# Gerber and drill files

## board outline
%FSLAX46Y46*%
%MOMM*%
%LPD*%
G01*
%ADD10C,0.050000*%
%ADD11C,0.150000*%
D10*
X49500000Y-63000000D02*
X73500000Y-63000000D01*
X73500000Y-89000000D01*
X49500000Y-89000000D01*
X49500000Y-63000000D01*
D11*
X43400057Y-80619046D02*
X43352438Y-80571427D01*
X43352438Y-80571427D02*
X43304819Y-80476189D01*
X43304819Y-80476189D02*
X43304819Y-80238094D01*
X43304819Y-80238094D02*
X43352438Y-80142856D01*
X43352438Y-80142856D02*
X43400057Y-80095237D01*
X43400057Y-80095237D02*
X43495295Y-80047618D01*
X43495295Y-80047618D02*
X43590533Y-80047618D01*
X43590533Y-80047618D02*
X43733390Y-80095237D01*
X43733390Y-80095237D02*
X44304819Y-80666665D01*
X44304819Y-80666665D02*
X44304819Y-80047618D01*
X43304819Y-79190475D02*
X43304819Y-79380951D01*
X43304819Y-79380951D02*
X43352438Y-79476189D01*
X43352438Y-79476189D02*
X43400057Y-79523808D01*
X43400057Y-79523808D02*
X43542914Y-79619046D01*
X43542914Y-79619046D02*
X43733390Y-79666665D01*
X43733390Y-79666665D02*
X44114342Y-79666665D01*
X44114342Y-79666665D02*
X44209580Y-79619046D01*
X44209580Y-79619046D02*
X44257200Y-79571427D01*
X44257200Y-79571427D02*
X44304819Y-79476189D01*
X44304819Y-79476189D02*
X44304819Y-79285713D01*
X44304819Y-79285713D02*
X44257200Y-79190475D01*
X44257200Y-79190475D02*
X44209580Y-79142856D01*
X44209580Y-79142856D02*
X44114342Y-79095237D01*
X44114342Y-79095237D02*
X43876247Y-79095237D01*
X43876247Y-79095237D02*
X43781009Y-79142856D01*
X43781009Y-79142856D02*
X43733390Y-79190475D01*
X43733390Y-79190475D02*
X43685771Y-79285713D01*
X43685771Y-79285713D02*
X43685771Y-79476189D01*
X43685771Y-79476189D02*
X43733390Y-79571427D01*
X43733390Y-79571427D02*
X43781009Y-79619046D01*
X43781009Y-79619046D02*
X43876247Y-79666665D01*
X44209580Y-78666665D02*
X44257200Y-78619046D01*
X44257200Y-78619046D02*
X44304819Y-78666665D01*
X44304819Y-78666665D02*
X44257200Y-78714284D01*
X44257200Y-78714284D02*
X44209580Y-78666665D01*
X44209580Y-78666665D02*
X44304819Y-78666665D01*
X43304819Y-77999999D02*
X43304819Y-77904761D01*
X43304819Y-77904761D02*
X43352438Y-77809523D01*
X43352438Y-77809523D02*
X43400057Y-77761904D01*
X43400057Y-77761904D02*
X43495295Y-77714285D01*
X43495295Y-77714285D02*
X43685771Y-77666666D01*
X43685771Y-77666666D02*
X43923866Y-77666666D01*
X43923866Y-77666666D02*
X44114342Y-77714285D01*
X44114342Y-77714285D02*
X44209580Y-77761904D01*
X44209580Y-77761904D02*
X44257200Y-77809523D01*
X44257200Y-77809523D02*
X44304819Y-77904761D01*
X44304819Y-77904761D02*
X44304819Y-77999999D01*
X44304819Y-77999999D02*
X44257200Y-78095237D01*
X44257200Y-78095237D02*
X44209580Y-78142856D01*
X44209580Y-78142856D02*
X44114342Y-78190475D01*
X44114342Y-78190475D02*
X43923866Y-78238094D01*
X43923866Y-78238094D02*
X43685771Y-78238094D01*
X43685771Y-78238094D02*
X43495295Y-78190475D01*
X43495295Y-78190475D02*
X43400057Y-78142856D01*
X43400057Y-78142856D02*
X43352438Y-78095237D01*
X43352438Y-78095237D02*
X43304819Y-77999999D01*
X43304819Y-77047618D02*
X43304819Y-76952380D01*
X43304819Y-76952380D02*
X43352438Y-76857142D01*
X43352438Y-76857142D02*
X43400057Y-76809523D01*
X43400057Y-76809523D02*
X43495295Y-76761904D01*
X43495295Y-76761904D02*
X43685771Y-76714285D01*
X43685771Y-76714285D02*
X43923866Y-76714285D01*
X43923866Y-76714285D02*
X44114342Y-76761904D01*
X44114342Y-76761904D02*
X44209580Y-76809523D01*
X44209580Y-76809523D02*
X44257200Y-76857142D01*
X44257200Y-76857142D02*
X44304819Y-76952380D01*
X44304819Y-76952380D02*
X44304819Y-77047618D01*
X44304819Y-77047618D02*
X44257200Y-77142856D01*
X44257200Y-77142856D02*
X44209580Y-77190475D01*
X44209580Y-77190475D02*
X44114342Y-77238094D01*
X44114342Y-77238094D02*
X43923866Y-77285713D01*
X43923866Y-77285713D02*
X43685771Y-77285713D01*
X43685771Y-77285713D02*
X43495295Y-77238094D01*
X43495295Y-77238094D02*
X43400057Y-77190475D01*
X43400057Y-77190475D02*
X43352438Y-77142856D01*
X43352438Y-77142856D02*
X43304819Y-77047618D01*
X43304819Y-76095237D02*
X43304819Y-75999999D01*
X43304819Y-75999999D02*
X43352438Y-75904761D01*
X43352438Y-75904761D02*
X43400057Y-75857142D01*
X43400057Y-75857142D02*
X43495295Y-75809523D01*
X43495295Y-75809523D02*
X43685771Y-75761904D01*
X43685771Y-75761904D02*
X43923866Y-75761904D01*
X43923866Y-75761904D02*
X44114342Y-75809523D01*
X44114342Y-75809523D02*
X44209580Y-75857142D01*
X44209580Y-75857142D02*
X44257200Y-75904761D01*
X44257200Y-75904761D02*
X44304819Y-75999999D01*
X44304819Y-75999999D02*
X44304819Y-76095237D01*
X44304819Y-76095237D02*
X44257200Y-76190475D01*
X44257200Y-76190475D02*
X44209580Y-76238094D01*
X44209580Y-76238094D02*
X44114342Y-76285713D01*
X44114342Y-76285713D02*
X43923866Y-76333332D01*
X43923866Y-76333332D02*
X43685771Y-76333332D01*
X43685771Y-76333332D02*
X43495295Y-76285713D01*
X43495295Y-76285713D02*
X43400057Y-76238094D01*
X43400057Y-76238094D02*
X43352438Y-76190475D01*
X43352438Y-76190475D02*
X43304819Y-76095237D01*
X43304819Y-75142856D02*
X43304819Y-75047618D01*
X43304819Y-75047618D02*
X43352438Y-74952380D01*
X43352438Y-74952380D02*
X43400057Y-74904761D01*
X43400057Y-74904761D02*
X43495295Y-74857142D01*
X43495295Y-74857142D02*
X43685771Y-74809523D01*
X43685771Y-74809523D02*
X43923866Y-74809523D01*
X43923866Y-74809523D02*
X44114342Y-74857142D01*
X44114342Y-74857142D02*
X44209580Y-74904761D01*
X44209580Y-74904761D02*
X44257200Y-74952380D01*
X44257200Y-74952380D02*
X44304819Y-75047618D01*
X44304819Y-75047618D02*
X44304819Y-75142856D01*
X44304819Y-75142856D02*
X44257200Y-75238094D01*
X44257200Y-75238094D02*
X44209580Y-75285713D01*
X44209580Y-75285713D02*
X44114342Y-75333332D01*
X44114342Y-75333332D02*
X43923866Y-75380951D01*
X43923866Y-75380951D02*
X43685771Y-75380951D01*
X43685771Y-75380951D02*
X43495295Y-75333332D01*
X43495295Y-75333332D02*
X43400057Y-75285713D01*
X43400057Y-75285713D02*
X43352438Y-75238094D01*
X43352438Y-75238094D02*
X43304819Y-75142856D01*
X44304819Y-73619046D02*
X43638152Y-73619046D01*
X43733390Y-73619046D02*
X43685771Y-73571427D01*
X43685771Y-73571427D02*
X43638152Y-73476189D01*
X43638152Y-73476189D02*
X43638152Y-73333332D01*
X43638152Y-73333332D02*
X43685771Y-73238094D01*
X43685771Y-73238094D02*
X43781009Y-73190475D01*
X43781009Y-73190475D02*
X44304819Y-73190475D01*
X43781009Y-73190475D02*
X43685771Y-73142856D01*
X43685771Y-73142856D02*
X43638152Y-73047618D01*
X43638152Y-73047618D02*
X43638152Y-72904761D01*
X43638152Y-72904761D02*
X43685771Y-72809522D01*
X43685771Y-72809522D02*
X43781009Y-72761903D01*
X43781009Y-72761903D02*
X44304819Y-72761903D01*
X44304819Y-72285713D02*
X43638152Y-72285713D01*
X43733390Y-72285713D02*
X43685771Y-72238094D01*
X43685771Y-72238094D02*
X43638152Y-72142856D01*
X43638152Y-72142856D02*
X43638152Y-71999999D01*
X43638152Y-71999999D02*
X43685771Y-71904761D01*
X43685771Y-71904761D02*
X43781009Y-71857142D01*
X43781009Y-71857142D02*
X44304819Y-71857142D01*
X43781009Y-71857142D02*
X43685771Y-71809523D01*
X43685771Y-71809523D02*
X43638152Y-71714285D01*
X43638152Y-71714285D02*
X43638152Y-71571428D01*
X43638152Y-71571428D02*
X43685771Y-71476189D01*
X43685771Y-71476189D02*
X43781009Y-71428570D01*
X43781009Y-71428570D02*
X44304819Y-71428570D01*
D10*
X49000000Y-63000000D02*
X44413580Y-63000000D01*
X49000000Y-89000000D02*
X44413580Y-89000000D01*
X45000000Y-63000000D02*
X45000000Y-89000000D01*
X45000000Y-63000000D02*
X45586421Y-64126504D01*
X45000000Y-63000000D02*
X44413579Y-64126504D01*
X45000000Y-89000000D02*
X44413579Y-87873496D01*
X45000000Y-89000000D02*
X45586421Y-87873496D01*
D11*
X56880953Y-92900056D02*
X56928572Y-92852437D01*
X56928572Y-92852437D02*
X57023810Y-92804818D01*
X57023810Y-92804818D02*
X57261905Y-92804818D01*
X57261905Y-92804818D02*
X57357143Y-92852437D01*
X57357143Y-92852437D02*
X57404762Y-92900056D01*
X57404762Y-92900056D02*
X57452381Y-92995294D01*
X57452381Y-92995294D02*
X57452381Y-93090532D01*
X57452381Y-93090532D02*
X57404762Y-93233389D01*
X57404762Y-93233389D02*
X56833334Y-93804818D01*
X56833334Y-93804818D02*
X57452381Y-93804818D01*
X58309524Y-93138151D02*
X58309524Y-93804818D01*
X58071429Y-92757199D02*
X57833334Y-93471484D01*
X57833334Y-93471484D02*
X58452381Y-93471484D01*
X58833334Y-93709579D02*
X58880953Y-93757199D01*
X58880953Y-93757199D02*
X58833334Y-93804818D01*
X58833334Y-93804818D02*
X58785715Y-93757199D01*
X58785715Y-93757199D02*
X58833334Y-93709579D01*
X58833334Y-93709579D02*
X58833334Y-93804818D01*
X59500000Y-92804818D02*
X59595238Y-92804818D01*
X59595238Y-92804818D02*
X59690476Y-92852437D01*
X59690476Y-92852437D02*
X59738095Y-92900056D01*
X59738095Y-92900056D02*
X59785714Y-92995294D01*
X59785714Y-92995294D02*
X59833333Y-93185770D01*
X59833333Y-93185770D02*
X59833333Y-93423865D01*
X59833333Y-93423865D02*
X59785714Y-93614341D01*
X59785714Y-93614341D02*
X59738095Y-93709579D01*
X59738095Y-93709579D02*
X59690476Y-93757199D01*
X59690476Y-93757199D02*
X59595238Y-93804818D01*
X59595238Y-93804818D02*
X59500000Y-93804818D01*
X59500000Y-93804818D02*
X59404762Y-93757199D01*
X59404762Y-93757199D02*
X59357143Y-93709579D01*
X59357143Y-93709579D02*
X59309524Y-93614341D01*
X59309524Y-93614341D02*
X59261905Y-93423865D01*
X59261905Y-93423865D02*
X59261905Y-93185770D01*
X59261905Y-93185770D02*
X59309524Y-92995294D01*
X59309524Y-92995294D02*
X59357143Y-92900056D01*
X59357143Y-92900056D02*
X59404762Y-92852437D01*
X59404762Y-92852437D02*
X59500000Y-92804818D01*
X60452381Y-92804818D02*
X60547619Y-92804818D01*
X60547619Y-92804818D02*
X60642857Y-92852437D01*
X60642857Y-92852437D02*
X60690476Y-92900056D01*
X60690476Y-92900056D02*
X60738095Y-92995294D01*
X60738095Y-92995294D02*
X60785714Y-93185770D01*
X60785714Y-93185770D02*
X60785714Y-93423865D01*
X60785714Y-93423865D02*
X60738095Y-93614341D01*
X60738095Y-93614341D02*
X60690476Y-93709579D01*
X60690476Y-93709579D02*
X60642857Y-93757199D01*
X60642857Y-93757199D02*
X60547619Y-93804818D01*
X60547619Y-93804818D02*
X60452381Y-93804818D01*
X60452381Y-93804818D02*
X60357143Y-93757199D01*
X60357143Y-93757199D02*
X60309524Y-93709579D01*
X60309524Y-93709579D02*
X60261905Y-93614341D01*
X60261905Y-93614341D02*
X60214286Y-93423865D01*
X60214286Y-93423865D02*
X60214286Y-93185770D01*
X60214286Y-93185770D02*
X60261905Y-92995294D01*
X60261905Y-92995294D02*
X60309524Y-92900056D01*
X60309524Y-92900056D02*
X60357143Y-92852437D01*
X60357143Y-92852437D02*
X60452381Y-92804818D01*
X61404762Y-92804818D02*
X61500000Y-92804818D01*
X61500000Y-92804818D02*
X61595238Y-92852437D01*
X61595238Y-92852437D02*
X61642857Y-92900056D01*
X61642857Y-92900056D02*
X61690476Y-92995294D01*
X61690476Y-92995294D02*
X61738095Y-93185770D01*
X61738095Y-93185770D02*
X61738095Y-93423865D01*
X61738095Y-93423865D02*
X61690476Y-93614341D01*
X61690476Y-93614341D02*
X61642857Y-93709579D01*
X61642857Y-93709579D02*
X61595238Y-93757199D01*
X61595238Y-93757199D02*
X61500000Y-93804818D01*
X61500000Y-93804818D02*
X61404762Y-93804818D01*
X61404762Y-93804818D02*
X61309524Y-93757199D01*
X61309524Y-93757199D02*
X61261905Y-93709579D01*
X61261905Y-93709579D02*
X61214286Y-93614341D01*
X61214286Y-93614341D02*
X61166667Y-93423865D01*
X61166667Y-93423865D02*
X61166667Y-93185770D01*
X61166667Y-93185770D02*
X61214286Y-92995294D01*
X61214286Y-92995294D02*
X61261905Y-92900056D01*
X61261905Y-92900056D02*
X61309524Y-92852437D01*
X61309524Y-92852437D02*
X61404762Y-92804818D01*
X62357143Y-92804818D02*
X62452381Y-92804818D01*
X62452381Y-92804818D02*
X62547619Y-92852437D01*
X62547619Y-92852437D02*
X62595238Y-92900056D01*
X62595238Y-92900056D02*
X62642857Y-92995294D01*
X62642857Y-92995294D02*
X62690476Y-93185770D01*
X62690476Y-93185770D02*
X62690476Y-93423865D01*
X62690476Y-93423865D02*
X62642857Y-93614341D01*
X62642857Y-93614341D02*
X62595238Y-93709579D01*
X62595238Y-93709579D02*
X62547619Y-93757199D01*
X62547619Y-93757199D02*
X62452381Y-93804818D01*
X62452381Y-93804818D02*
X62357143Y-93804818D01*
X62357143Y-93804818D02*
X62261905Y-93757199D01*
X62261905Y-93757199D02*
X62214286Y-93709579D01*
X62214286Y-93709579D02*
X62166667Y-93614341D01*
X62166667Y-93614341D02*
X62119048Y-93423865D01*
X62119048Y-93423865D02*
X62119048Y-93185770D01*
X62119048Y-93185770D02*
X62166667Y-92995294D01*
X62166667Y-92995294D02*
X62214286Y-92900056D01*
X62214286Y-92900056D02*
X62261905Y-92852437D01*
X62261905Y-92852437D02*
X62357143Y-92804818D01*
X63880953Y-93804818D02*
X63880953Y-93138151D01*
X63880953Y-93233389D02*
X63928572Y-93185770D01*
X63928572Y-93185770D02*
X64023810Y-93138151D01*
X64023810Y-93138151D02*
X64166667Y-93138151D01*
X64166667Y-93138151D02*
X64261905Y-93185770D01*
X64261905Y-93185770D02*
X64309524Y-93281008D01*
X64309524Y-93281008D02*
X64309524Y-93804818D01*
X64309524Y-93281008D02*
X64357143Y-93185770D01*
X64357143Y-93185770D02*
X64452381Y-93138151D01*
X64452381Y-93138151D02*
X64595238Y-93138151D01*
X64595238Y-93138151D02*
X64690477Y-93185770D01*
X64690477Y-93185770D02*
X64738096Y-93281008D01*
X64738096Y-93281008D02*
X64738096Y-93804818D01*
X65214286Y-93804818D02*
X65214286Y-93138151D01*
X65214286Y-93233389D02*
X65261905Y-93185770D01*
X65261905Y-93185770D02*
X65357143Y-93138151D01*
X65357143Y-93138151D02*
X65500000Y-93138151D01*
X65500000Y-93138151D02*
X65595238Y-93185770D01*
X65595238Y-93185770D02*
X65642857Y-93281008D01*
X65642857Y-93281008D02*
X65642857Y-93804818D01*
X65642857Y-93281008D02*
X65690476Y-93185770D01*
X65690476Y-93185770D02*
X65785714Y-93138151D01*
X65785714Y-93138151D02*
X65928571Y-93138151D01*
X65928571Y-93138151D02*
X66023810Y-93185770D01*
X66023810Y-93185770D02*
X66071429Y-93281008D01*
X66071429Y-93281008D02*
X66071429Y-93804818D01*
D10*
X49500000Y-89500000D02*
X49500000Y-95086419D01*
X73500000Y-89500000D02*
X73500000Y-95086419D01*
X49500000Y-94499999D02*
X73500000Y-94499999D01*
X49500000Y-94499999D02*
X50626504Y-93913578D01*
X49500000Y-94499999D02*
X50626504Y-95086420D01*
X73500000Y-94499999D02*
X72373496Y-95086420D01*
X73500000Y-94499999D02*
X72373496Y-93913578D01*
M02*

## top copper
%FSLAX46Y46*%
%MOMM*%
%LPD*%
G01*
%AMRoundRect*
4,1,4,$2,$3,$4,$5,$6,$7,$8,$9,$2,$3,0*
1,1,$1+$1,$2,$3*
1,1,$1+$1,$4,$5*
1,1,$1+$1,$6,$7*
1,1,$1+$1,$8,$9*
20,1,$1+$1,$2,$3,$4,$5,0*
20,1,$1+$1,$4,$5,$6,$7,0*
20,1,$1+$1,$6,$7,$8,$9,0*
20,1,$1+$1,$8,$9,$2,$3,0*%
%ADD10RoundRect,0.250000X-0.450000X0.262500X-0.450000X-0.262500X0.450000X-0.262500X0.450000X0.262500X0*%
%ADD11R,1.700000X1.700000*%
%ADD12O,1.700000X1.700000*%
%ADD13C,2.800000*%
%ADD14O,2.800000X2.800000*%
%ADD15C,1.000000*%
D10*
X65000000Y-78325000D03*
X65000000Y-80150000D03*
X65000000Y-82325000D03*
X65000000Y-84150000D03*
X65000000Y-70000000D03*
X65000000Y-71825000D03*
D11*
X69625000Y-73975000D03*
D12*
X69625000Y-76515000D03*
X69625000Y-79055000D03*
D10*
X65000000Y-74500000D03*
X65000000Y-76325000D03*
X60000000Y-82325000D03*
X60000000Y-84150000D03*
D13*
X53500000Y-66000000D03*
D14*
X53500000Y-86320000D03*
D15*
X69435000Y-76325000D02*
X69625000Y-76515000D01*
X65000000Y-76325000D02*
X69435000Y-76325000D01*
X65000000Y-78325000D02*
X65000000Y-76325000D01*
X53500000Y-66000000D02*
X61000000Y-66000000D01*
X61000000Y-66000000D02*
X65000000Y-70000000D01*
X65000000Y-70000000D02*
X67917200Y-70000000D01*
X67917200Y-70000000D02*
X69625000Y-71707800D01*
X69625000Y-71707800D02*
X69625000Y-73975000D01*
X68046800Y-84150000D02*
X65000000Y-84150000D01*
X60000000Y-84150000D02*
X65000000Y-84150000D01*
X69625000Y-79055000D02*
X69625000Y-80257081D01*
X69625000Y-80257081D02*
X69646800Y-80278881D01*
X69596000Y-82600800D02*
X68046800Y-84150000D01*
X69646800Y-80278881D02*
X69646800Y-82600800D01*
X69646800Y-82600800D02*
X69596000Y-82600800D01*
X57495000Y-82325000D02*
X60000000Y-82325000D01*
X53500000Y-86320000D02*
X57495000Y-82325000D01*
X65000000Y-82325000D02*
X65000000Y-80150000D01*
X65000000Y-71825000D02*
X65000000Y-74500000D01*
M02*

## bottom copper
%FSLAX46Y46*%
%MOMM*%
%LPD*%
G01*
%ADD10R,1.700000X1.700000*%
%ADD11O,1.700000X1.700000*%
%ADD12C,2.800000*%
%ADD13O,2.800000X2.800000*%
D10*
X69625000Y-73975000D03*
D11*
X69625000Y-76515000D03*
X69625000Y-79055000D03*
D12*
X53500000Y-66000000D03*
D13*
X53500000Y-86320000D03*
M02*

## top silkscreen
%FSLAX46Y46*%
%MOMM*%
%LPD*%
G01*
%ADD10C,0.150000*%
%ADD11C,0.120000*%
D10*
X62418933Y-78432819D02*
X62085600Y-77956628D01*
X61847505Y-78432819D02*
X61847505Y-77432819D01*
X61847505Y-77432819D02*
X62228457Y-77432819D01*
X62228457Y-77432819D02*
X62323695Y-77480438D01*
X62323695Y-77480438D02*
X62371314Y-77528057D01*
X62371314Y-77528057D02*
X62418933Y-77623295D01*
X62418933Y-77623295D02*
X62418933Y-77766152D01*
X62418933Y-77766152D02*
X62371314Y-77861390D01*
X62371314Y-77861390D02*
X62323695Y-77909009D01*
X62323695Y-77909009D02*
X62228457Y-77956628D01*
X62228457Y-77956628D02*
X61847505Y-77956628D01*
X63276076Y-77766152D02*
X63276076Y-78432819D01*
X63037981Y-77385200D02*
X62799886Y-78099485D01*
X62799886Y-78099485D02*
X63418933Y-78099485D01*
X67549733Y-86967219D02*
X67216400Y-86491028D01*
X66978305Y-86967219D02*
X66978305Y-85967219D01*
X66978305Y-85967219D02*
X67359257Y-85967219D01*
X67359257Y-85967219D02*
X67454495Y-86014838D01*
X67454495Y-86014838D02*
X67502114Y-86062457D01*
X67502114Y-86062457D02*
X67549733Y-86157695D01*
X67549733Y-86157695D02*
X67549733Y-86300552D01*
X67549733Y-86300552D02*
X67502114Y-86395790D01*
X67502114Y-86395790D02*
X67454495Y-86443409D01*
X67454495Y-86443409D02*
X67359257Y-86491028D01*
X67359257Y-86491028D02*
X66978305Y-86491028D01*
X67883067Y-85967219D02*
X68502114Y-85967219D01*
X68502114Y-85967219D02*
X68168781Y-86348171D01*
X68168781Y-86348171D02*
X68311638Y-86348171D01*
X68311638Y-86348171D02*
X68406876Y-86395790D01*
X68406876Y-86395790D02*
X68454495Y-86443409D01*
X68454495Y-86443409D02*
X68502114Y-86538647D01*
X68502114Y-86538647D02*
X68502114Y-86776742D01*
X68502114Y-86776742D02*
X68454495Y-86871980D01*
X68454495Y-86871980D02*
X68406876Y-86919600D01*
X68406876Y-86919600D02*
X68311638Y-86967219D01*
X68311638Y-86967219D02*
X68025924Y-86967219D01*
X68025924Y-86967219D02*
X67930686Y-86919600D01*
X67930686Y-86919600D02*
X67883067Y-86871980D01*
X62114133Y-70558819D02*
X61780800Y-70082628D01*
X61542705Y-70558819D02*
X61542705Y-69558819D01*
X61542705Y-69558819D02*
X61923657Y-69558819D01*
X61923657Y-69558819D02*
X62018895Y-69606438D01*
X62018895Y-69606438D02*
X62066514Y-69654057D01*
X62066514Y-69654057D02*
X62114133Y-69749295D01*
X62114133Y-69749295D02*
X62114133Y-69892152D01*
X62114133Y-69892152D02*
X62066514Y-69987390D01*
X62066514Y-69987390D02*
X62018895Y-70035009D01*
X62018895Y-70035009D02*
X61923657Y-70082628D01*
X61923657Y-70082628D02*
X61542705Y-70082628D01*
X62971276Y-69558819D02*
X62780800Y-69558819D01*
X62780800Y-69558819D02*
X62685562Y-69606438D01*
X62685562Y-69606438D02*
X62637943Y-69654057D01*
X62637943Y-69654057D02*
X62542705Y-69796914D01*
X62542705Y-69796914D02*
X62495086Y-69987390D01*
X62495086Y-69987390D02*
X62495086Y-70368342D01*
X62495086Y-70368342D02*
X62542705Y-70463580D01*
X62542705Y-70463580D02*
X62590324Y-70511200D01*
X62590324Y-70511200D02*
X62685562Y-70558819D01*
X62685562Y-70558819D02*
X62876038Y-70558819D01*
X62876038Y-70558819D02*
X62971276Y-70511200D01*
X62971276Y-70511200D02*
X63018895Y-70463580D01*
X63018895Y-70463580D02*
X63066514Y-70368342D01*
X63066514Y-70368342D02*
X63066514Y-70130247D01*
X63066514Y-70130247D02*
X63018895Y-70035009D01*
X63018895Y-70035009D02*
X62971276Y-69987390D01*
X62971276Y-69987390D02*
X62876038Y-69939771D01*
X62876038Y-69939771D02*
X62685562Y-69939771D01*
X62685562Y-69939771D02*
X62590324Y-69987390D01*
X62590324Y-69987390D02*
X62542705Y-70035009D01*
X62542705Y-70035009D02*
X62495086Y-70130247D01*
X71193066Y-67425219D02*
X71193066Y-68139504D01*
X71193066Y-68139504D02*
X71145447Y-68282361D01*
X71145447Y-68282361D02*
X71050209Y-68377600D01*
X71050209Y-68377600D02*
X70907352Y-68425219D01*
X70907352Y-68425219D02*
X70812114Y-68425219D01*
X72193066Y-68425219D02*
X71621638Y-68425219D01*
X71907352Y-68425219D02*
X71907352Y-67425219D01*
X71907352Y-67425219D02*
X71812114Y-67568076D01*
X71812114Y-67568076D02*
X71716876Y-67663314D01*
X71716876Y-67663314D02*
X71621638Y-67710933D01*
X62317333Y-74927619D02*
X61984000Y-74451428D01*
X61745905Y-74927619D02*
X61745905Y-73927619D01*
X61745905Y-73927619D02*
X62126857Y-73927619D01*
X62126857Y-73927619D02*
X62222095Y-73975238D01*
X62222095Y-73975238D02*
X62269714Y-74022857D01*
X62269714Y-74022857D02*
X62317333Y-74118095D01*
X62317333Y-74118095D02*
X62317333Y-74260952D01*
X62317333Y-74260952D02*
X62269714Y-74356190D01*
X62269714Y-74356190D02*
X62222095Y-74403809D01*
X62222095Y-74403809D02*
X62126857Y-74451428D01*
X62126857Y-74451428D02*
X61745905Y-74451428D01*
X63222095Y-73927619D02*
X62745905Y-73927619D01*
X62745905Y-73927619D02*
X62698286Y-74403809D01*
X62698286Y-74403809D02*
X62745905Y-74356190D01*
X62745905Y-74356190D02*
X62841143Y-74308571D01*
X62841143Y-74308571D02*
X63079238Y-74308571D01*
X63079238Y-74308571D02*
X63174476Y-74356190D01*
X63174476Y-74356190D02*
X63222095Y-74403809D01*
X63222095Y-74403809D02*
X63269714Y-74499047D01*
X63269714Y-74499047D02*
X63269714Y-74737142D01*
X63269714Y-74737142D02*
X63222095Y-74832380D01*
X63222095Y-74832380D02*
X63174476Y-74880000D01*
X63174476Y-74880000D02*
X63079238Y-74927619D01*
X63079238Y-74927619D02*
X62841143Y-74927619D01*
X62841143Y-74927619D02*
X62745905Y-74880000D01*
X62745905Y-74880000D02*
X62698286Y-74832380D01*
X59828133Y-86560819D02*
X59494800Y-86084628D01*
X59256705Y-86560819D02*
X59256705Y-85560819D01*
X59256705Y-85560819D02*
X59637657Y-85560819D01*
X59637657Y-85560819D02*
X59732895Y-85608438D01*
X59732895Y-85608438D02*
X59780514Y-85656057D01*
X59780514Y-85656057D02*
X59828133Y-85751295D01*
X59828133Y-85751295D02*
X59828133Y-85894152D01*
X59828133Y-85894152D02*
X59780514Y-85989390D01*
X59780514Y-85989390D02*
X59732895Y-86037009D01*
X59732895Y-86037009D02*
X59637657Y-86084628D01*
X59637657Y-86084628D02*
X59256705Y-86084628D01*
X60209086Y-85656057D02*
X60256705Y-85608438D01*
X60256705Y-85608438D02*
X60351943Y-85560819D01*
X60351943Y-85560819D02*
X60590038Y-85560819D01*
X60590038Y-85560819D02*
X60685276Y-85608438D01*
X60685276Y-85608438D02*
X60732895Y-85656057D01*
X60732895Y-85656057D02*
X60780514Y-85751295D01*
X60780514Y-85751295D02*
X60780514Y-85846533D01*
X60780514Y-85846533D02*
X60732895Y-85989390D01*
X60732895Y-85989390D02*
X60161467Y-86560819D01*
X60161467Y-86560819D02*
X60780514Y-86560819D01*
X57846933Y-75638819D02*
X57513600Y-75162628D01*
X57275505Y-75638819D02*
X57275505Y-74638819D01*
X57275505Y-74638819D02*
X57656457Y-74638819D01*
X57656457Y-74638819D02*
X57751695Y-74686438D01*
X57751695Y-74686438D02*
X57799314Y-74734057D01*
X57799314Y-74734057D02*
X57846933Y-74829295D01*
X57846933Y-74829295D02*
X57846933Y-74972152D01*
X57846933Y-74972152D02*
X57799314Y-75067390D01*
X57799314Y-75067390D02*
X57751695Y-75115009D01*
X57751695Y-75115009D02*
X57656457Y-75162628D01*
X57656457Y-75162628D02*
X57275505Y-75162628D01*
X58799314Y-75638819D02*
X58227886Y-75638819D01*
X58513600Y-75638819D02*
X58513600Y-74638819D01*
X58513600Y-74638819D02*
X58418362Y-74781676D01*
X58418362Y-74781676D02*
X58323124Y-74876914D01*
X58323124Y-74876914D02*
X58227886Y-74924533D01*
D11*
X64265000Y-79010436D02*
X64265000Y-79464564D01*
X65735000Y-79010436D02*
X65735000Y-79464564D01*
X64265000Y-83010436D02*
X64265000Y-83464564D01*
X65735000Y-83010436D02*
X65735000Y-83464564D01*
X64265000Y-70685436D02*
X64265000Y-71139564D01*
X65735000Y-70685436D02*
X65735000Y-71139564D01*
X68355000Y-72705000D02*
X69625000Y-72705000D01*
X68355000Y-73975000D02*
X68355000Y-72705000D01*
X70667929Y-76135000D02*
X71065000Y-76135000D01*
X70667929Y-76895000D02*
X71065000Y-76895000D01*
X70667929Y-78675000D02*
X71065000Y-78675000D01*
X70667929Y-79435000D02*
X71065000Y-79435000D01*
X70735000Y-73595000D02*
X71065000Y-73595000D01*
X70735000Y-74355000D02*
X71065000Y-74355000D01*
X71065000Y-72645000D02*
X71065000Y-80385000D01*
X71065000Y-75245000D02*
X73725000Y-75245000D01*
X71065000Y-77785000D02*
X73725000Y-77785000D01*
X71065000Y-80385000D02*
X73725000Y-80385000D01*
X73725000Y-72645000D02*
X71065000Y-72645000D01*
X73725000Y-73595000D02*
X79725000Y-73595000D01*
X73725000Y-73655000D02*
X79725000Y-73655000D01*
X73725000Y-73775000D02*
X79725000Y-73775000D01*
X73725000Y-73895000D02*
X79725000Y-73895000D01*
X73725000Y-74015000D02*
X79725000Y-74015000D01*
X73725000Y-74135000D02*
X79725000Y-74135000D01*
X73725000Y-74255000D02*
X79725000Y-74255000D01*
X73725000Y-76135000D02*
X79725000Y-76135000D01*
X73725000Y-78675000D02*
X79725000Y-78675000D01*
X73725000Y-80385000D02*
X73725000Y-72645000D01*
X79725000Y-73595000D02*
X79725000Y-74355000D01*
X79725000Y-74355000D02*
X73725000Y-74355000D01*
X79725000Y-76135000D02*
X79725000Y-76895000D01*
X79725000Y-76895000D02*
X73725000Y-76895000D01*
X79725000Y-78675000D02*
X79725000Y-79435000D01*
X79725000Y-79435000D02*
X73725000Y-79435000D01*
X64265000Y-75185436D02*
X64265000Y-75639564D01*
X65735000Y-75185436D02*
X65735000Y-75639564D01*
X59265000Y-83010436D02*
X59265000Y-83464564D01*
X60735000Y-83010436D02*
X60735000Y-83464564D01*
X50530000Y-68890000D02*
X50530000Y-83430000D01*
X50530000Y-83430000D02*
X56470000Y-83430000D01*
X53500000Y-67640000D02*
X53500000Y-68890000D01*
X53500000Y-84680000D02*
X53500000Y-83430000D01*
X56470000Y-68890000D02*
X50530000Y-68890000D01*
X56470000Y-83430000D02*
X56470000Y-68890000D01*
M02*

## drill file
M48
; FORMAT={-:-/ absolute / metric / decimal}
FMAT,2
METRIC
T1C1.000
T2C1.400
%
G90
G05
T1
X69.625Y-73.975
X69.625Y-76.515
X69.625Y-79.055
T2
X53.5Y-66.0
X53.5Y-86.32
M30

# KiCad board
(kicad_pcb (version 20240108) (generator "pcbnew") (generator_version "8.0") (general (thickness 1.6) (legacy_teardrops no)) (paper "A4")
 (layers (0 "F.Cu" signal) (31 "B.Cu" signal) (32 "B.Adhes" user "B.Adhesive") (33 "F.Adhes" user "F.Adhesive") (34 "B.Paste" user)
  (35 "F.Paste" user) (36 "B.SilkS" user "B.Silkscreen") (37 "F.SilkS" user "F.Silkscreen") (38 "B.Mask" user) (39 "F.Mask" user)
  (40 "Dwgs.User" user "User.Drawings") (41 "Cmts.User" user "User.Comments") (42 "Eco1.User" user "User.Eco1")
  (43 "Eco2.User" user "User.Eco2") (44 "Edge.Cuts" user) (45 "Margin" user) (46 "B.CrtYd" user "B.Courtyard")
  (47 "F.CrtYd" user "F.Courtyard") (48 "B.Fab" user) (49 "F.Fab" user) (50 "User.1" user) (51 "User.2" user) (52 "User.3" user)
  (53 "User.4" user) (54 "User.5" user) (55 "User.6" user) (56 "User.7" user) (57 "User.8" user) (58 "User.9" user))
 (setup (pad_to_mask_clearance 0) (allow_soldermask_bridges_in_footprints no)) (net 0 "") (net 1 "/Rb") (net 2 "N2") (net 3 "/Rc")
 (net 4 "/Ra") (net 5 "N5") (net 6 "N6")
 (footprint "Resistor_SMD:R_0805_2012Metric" (layer "F.Cu") (at 65 79.2375 -90)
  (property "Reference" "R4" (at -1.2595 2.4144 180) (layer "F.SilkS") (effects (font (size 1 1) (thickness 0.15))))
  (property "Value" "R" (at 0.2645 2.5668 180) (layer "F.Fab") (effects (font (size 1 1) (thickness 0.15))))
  (fp_line (start -0.227064 0.735) (end 0.227064 0.735) (stroke (width 0.12) (type solid)) (layer "F.SilkS"))
  (fp_line (start -0.227064 -0.735) (end 0.227064 -0.735) (stroke (width 0.12) (type solid)) (layer "F.SilkS"))
  (pad "1" smd roundrect (at -0.9125 0 270) (size 1.025 1.4) (layers "F.Cu" "F.Paste" "F.Mask") (roundrect_rratio 0.243902) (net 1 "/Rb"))
  (pad "2" smd roundrect (at 0.9125 0 270) (size 1.025 1.4) (layers "F.Cu" "F.Paste" "F.Mask") (roundrect_rratio 0.243902) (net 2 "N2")))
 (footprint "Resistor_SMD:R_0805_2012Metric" (layer "F.Cu") (at 65 83.2375 -90)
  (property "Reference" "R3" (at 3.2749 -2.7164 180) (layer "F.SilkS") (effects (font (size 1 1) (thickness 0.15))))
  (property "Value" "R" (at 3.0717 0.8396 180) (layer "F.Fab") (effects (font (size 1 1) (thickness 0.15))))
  (fp_line (start -0.227064 0.735) (end 0.227064 0.735) (stroke (width 0.12) (type solid)) (layer "F.SilkS"))
  (fp_line (start -0.227064 -0.735) (end 0.227064 -0.735) (stroke (width 0.12) (type solid)) (layer "F.SilkS"))
  (pad "1" smd roundrect (at -0.9125 0 270) (size 1.025 1.4) (layers "F.Cu" "F.Paste" "F.Mask") (roundrect_rratio 0.243902) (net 2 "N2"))
  (pad "2" smd roundrect (at 0.9125 0 270) (size 1.025 1.4) (layers "F.Cu" "F.Paste" "F.Mask") (roundrect_rratio 0.243902) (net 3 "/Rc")))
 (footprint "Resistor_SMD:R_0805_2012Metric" (layer "F.Cu") (at 65 70.9125 -90)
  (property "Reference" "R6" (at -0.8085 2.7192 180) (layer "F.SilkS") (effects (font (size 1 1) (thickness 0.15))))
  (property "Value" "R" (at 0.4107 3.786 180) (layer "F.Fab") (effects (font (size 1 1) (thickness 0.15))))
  (fp_line (start -0.227064 0.735) (end 0.227064 0.735) (stroke (width 0.12) (type solid)) (layer "F.SilkS"))
  (fp_line (start -0.227064 -0.735) (end 0.227064 -0.735) (stroke (width 0.12) (type solid)) (layer "F.SilkS"))
  (pad "1" smd roundrect (at -0.9125 0 270) (size 1.025 1.4) (layers "F.Cu" "F.Paste" "F.Mask") (roundrect_rratio 0.243902) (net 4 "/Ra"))
  (pad "2" smd roundrect (at 0.9125 0 270) (size 1.025 1.4) (layers "F.Cu" "F.Paste" "F.Mask") (roundrect_rratio 0.243902) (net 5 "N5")))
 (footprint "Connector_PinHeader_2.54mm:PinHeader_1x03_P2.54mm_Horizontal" (layer "F.Cu") (at 69.625 73.975)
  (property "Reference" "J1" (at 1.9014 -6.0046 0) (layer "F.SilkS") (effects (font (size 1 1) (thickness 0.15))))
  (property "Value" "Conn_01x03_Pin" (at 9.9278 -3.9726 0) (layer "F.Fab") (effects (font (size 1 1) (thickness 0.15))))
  (fp_line (start -1.27 -1.27) (end 0 -1.27) (stroke (width 0.12) (type solid)) (layer "F.SilkS"))
  (fp_line (start -1.27 0) (end -1.27 -1.27) (stroke (width 0.12) (type solid)) (layer "F.SilkS"))
  (fp_line (start 1.042929 2.16) (end 1.44 2.16) (stroke (width 0.12) (type solid)) (layer "F.SilkS"))
  (fp_line (start 1.042929 2.92) (end 1.44 2.92) (stroke (width 0.12) (type solid)) (layer "F.SilkS"))
  (fp_line (start 1.042929 4.7) (end 1.44 4.7) (stroke (width 0.12) (type solid)) (layer "F.SilkS"))
  (fp_line (start 1.042929 5.46) (end 1.44 5.46) (stroke (width 0.12) (type solid)) (layer "F.SilkS"))
  (fp_line (start 1.11 -0.38) (end 1.44 -0.38) (stroke (width 0.12) (type solid)) (layer "F.SilkS"))
  (fp_line (start 1.11 0.38) (end 1.44 0.38) (stroke (width 0.12) (type solid)) (layer "F.SilkS"))
  (fp_line (start 1.44 -1.33) (end 1.44 6.41) (stroke (width 0.12) (type solid)) (layer "F.SilkS"))
  (fp_line (start 1.44 1.27) (end 4.1 1.27) (stroke (width 0.12) (type solid)) (layer "F.SilkS"))
  (fp_line (start 1.44 3.81) (end 4.1 3.81) (stroke (width 0.12) (type solid)) (layer "F.SilkS"))
  (fp_line (start 1.44 6.41) (end 4.1 6.41) (stroke (width 0.12) (type solid)) (layer "F.SilkS"))
  (fp_line (start 4.1 -1.33) (end 1.44 -1.33) (stroke (width 0.12) (type solid)) (layer "F.SilkS"))
  (fp_line (start 4.1 -0.38) (end 10.1 -0.38) (stroke (width 0.12) (type solid)) (layer "F.SilkS"))
  (fp_line (start 4.1 -0.32) (end 10.1 -0.32) (stroke (width 0.12) (type solid)) (layer "F.SilkS"))
  (fp_line (start 4.1 -0.2) (end 10.1 -0.2) (stroke (width 0.12) (type solid)) (layer "F.SilkS"))
  (fp_line (start 4.1 -0.08) (end 10.1 -0.08) (stroke (width 0.12) (type solid)) (layer "F.SilkS"))
  (fp_line (start 4.1 0.04) (end 10.1 0.04) (stroke (width 0.12) (type solid)) (layer "F.SilkS"))
  (fp_line (start 4.1 0.16) (end 10.1 0.16) (stroke (width 0.12) (type solid)) (layer "F.SilkS"))
  (fp_line (start 4.1 0.28) (end 10.1 0.28) (stroke (width 0.12) (type solid)) (layer "F.SilkS"))
  (fp_line (start 4.1 2.16) (end 10.1 2.16) (stroke (width 0.12) (type solid)) (layer "F.SilkS"))
  (fp_line (start 4.1 4.7) (end 10.1 4.7) (stroke (width 0.12) (type solid)) (layer "F.SilkS"))
  (fp_line (start 4.1 6.41) (end 4.1 -1.33) (stroke (width 0.12) (type solid)) (layer "F.SilkS"))
  (fp_line (start 10.1 -0.38) (end 10.1 0.38) (stroke (width 0.12) (type solid)) (layer "F.SilkS"))
  (fp_line (start 10.1 0.38) (end 4.1 0.38) (stroke (width 0.12) (type solid)) (layer "F.SilkS"))
  (fp_line (start 10.1 2.16) (end 10.1 2.92) (stroke (width 0.12) (type solid)) (layer "F.SilkS"))
  (fp_line (start 10.1 2.92) (end 4.1 2.92) (stroke (width 0.12) (type solid)) (layer "F.SilkS"))
  (fp_line (start 10.1 4.7) (end 10.1 5.46) (stroke (width 0.12) (type solid)) (layer "F.SilkS"))
  (fp_line (start 10.1 5.46) (end 4.1 5.46) (stroke (width 0.12) (type solid)) (layer "F.SilkS"))
  (pad "1" thru_hole rect (at 0 0) (size 1.7 1.7) (drill 1) (layers "*.Cu" "*.Mask") (remove_unused_layers no) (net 4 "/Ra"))
  (pad "2" thru_hole oval (at 0 2.54) (size 1.7 1.7) (drill 1) (layers "*.Cu" "*.Mask") (remove_unused_layers no) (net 1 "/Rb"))
  (pad "3" thru_hole oval (at 0 5.08) (size 1.7 1.7) (drill 1) (layers "*.Cu" "*.Mask") (remove_unused_layers no) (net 3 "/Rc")))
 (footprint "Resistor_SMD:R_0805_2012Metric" (layer "F.Cu") (at 65 75.4125 -90)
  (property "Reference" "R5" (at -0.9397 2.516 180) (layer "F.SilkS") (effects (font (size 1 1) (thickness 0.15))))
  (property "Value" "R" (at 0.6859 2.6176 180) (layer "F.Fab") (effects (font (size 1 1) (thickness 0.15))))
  (fp_line (start -0.227064 0.735) (end 0.227064 0.735) (stroke (width 0.12) (type solid)) (layer "F.SilkS"))
  (fp_line (start -0.227064 -0.735) (end 0.227064 -0.735) (stroke (width 0.12) (type solid)) (layer "F.SilkS"))
  (pad "1" smd roundrect (at -0.9125 0 270) (size 1.025 1.4) (layers "F.Cu" "F.Paste" "F.Mask") (roundrect_rratio 0.243902) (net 5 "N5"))
  (pad "2" smd roundrect (at 0.9125 0 270) (size 1.025 1.4) (layers "F.Cu" "F.Paste" "F.Mask") (roundrect_rratio 0.243902) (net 1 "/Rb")))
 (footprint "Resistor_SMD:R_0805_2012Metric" (layer "F.Cu") (at 60 83.2375 -90)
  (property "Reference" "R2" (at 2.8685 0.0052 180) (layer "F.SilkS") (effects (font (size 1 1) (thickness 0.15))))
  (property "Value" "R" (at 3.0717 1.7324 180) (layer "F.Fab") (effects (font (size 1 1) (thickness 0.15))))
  (fp_line (start -0.227064 0.735) (end 0.227064 0.735) (stroke (width 0.12) (type solid)) (layer "F.SilkS"))
  (fp_line (start -0.227064 -0.735) (end 0.227064 -0.735) (stroke (width 0.12) (type solid)) (layer "F.SilkS"))
  (pad "1" smd roundrect (at -0.9125 0 270) (size 1.025 1.4) (layers "F.Cu" "F.Paste" "F.Mask") (roundrect_rratio 0.243902) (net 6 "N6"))
  (pad "2" smd roundrect (at 0.9125 0 270) (size 1.025 1.4) (layers "F.Cu" "F.Paste" "F.Mask") (roundrect_rratio 0.243902) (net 3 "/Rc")))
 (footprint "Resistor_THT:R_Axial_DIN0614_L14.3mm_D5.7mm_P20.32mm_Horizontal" (layer "F.Cu") (at 53.5 66 -90)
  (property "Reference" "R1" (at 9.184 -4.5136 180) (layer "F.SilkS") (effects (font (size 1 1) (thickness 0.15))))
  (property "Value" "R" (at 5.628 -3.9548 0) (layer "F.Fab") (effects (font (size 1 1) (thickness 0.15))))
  (fp_line (start 2.89 2.97) (end 17.43 2.97) (stroke (width 0.12) (type solid)) (layer "F.SilkS"))
  (fp_line (start 17.43 2.97) (end 17.43 -2.97) (stroke (width 0.12) (type solid)) (layer "F.SilkS"))
  (fp_line (start 1.64 0) (end 2.89 0) (stroke (width 0.12) (type solid)) (layer "F.SilkS"))
  (fp_line (start 18.68 0) (end 17.43 0) (stroke (width 0.12) (type solid)) (layer "F.SilkS"))
  (fp_line (start 2.89 -2.97) (end 2.89 2.97) (stroke (width 0.12) (type solid)) (layer "F.SilkS"))
  (fp_line (start 17.43 -2.97) (end 2.89 -2.97) (stroke (width 0.12) (type solid)) (layer "F.SilkS"))
  (pad "1" thru_hole circle (at 0 0 270) (size 2.8 2.8) (drill 1.4) (layers "*.Cu" "*.Mask") (remove_unused_layers no) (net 4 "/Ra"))
  (pad "2" thru_hole oval (at 20.32 0 270) (size 2.8 2.8) (drill 1.4) (layers "*.Cu" "*.Mask") (remove_unused_layers no) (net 6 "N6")))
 (gr_rect (start 49.5 63) (end 73.5 89) (stroke (width 0.05) (type default)) (fill none) (layer "Edge.Cuts"))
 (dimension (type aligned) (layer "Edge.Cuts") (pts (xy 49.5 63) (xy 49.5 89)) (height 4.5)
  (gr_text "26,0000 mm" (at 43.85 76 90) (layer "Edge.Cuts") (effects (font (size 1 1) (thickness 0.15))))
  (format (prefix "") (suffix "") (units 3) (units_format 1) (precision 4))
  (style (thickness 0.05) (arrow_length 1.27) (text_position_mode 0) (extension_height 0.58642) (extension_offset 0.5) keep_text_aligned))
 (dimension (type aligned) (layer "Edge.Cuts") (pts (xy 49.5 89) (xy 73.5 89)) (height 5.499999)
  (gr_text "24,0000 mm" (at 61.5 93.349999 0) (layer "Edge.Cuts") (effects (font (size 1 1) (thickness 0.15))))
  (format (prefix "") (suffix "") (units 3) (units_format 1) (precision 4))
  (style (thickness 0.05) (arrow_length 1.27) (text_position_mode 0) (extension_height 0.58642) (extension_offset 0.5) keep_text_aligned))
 (segment (start 69.435 76.325) (end 69.625 76.515) (width 1) (layer "F.Cu") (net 1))
 (segment (start 65 76.325) (end 69.435 76.325) (width 1) (layer "F.Cu") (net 1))
 (segment (start 65 78.325) (end 65 76.325) (width 1) (layer "F.Cu") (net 1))
 (segment (start 53.5 66) (end 61 66) (width 1) (layer "F.Cu") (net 4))
 (segment (start 61 66) (end 65 70) (width 1) (layer "F.Cu") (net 4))
 (segment (start 65 70) (end 67.9172 70) (width 1) (layer "F.Cu") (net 4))
 (segment (start 67.9172 70) (end 69.625 71.7078) (width 1) (layer "F.Cu") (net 4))
 (segment (start 69.625 71.7078) (end 69.625 73.975) (width 1) (layer "F.Cu") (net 4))
 (segment (start 68.0468 84.15) (end 65 84.15) (width 1) (layer "F.Cu") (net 3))
 (segment (start 60 84.15) (end 65 84.15) (width 1) (layer "F.Cu") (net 3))
 (segment (start 69.625 79.055) (end 69.625 80.257081) (width 1) (layer "F.Cu") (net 3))
 (segment (start 69.625 80.257081) (end 69.6468 80.278881) (width 1) (layer "F.Cu") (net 3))
 (segment (start 69.596 82.6008) (end 68.0468 84.15) (width 1) (layer "F.Cu") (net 3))
 (segment (start 69.6468 80.278881) (end 69.6468 82.6008) (width 1) (layer "F.Cu") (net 3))
 (segment (start 69.6468 82.6008) (end 69.596 82.6008) (width 1) (layer "F.Cu") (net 3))
 (segment (start 57.495 82.325) (end 60 82.325) (width 1) (layer "F.Cu") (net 6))
 (segment (start 53.5 86.32) (end 57.495 82.325) (width 1) (layer "F.Cu") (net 6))
 (segment (start 65 82.325) (end 65 80.15) (width 1) (layer "F.Cu") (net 2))
 (segment (start 65 71.825) (end 65 74.5) (width 1) (layer "F.Cu") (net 5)))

